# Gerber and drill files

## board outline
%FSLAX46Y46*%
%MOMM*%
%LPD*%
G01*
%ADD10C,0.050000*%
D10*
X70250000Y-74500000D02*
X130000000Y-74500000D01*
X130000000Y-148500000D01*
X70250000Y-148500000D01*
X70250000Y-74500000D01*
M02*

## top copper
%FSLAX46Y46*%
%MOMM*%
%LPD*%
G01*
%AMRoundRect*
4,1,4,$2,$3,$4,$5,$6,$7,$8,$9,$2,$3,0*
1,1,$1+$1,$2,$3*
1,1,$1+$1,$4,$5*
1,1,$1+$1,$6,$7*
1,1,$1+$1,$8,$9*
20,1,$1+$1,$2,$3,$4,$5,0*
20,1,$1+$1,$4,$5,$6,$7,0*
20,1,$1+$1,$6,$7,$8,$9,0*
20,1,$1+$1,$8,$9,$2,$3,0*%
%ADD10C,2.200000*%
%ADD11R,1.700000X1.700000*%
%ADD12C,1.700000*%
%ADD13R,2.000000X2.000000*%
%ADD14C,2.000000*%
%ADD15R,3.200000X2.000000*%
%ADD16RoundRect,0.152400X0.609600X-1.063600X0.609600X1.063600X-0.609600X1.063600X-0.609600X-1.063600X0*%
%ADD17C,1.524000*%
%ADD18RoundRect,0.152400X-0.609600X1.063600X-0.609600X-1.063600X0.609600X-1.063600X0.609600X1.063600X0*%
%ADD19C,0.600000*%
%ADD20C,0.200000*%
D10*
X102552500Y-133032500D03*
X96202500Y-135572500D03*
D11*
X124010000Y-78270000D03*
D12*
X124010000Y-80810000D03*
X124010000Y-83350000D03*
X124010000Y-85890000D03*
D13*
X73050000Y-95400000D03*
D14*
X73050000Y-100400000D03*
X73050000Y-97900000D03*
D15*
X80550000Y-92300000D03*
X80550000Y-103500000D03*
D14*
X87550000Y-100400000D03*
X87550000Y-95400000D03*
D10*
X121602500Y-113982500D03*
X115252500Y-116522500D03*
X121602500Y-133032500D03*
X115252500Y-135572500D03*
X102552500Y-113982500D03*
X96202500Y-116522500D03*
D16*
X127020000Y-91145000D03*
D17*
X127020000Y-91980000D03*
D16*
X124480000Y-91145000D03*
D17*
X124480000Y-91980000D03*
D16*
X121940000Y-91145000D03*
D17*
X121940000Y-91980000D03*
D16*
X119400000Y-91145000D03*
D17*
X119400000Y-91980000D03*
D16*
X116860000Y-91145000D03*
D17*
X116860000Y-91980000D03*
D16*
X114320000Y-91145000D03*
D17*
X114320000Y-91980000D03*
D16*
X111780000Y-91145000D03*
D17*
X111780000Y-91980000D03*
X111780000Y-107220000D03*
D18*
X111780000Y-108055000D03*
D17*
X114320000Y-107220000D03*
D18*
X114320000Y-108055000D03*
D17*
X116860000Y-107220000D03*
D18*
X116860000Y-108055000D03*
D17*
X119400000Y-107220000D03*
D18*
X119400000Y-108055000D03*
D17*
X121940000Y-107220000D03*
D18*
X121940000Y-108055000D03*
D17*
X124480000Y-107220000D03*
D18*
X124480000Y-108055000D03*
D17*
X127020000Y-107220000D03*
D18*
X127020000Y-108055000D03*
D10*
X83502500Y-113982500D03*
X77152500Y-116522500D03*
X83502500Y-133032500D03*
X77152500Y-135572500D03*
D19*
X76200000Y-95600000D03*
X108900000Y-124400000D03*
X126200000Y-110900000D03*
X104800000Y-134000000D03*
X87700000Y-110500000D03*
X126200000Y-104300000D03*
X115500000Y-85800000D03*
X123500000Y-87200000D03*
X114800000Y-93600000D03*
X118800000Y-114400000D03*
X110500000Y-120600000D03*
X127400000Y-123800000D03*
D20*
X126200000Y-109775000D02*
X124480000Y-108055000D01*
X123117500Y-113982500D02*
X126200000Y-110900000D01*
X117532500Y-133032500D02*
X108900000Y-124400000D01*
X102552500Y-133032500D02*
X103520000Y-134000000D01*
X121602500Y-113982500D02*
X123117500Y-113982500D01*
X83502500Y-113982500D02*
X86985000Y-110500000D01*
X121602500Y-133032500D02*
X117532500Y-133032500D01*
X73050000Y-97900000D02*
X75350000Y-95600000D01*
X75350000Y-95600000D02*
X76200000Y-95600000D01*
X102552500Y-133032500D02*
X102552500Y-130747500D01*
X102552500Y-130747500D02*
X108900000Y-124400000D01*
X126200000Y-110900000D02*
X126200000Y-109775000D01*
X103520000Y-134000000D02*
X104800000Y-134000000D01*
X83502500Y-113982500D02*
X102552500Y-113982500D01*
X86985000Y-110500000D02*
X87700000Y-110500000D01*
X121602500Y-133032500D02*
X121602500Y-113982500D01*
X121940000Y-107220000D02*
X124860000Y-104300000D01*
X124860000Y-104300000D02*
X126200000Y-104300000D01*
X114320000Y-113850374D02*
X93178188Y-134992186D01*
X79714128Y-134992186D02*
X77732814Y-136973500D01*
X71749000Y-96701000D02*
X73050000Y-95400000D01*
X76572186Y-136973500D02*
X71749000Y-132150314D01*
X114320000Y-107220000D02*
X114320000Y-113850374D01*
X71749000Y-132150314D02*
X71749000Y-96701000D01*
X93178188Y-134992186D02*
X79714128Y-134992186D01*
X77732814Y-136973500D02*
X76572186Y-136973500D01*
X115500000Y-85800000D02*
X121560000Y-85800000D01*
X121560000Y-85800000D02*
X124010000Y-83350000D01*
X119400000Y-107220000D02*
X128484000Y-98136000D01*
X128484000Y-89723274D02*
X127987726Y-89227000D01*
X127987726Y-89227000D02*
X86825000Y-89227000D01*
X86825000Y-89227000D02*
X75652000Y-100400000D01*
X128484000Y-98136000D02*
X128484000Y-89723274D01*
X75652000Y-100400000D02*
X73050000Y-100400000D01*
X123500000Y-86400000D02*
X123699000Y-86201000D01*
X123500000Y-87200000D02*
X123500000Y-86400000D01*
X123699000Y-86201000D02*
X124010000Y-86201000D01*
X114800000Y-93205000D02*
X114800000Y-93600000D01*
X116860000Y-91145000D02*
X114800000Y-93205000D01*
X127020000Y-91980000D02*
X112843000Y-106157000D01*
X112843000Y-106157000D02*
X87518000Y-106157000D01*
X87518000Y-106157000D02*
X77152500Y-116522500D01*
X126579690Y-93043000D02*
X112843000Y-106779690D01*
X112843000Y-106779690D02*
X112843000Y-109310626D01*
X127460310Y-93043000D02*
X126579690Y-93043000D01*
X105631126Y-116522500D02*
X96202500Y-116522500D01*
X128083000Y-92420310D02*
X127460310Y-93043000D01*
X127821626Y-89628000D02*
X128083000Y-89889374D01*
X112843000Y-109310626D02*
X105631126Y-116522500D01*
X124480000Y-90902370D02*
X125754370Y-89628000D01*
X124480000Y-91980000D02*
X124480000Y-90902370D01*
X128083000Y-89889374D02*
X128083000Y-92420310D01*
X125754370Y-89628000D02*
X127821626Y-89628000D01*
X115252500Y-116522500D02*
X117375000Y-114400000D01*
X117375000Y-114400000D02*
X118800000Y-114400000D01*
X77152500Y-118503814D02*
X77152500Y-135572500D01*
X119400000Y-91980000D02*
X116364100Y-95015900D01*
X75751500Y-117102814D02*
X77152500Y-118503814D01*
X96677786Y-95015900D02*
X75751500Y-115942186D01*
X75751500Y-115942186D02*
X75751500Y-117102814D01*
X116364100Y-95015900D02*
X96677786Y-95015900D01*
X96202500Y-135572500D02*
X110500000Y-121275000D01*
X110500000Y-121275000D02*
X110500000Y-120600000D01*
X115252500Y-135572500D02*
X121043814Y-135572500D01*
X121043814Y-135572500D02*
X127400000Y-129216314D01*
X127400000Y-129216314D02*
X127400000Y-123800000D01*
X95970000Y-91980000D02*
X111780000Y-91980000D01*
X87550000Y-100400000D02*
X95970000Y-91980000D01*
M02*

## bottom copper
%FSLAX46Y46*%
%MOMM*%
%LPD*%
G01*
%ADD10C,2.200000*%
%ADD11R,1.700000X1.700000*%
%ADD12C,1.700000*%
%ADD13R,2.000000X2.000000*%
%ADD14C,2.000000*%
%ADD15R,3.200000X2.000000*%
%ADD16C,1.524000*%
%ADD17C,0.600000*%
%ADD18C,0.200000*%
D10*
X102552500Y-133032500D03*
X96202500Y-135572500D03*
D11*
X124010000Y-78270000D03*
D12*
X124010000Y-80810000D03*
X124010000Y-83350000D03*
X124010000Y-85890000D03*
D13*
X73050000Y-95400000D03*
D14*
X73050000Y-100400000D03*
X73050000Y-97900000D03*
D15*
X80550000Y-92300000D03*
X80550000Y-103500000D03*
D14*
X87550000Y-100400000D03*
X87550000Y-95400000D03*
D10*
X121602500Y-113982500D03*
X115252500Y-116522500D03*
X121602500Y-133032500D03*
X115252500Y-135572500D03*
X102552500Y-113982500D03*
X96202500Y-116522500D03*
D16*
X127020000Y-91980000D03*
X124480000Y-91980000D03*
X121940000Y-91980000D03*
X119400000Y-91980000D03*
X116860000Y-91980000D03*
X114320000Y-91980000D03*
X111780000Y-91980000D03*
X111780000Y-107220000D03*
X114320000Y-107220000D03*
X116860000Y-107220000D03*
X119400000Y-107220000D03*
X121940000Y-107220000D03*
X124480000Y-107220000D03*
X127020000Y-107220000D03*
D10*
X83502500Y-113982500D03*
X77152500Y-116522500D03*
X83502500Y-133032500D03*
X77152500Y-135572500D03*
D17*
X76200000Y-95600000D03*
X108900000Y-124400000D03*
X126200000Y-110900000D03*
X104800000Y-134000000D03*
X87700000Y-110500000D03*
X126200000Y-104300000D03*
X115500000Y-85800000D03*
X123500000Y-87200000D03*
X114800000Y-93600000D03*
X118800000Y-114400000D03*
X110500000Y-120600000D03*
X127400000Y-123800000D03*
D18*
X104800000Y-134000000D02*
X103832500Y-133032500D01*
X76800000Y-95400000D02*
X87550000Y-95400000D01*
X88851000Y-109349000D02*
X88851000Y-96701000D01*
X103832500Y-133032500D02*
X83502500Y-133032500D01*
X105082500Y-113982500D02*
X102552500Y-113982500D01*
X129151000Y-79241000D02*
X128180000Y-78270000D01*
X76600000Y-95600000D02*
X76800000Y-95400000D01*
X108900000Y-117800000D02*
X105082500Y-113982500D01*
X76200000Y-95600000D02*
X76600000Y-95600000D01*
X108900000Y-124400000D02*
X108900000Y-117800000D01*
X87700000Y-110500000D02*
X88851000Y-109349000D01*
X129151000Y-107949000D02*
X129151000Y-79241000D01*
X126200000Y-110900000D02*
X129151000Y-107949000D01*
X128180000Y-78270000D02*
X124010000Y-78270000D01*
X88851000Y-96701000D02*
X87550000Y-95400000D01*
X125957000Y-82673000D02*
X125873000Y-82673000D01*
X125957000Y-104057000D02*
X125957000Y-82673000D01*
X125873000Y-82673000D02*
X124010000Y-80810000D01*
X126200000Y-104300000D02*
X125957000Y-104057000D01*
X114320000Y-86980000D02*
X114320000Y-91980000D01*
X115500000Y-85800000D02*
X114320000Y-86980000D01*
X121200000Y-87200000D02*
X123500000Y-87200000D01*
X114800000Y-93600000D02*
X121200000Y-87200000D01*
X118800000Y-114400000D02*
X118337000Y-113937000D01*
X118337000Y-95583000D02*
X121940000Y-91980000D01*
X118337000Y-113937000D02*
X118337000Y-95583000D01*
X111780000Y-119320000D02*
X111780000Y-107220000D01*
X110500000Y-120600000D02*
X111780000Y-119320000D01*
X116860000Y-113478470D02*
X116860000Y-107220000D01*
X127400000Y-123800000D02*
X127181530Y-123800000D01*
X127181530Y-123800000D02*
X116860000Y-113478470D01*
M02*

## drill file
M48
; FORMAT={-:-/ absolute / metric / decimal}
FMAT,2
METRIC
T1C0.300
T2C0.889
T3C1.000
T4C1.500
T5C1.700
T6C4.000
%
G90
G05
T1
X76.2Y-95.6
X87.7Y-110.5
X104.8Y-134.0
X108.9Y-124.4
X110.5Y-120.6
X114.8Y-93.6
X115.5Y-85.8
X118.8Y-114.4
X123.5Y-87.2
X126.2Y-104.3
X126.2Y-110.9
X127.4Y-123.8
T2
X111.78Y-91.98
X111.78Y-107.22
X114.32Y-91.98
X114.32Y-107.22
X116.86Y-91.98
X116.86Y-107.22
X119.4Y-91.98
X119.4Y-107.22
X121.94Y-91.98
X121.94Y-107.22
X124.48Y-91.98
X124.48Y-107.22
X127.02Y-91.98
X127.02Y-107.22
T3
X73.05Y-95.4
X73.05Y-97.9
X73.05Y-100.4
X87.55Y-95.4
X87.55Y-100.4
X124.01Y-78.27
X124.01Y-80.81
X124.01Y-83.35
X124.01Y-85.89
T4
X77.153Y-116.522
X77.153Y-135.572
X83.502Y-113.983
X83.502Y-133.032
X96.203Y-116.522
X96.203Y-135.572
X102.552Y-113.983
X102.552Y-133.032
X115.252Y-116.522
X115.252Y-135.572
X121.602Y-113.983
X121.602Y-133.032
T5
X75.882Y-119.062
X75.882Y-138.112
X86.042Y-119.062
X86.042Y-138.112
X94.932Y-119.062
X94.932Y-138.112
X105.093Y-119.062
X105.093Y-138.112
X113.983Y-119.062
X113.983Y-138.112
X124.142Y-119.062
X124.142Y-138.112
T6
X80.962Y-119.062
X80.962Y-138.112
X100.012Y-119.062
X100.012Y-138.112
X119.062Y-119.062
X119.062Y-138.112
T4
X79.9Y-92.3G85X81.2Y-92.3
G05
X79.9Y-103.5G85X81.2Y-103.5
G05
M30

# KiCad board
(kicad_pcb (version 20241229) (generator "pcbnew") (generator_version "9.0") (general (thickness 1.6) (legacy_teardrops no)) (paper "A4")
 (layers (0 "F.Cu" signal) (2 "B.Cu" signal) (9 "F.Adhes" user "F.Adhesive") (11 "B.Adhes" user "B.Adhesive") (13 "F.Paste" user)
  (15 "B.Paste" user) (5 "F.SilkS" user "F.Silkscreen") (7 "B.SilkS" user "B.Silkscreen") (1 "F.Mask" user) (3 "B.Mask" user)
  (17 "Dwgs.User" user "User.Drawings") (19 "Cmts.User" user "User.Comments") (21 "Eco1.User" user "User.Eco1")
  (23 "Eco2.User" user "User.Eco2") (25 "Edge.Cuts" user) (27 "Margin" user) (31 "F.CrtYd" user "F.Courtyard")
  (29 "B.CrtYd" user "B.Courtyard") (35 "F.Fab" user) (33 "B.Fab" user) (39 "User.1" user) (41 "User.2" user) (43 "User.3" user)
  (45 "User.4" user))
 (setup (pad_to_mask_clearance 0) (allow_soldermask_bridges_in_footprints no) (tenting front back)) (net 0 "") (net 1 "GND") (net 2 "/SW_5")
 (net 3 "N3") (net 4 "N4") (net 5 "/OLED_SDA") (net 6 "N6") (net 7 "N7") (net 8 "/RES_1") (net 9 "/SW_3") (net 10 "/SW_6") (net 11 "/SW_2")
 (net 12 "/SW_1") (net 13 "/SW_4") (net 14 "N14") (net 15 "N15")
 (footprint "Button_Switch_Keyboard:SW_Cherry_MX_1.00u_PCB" (layer "F.Cu") (at 102.5525 133.0325)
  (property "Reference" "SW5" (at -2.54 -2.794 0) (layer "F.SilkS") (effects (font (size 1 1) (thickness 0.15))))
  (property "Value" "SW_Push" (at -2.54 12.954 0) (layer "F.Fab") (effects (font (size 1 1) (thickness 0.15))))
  (pad "" np_thru_hole circle (at -7.62 5.08) (size 1.7 1.7) (drill 1.7) (layers "*.Cu" "*.Mask"))
  (pad "" np_thru_hole circle (at -2.54 5.08) (size 4 4) (drill 4) (layers "*.Cu" "*.Mask"))
  (pad "" np_thru_hole circle (at 2.54 5.08) (size 1.7 1.7) (drill 1.7) (layers "*.Cu" "*.Mask"))
  (pad "1" thru_hole circle (at 0 0) (size 2.2 2.2) (drill 1.5) (layers "*.Cu" "*.Mask") (remove_unused_layers no) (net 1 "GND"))
  (pad "2" thru_hole circle (at -6.35 2.54) (size 2.2 2.2) (drill 1.5) (layers "*.Cu" "*.Mask") (remove_unused_layers no) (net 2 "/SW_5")))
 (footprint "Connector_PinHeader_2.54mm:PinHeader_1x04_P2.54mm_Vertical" (layer "F.Cu") (at 124.01 78.27)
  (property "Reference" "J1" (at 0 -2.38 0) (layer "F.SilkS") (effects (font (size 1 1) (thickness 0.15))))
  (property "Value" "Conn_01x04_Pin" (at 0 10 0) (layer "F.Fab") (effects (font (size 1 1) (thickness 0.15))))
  (pad "1" thru_hole rect (at 0 0) (size 1.7 1.7) (drill 1) (layers "*.Cu" "*.Mask") (remove_unused_layers no) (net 1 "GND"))
  (pad "2" thru_hole circle (at 0 2.54) (size 1.7 1.7) (drill 1) (layers "*.Cu" "*.Mask") (remove_unused_layers no) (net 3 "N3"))
  (pad "3" thru_hole circle (at 0 5.08) (size 1.7 1.7) (drill 1) (layers "*.Cu" "*.Mask") (remove_unused_layers no) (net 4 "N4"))
  (pad "4" thru_hole circle (at 0 7.62) (size 1.7 1.7) (drill 1) (layers "*.Cu" "*.Mask") (remove_unused_layers no) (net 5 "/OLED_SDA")))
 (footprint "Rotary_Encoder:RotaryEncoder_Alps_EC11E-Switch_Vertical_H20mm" (layer "F.Cu") (at 73.05 95.4)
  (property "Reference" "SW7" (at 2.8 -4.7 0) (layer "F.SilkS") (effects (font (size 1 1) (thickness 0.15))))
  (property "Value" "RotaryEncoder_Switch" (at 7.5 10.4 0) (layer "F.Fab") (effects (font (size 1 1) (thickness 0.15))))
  (pad "A" thru_hole rect (at 0 0) (size 2 2) (drill 1) (layers "*.Cu" "*.Mask") (remove_unused_layers no) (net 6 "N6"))
  (pad "B" thru_hole circle (at 0 5) (size 2 2) (drill 1) (layers "*.Cu" "*.Mask") (remove_unused_layers no) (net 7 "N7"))
  (pad "C" thru_hole circle (at 0 2.5) (size 2 2) (drill 1) (layers "*.Cu" "*.Mask") (remove_unused_layers no) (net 1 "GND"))
  (pad "MP" thru_hole rect (at 7.5 -3.1) (size 3.2 2) (drill oval 2.8 1.5) (layers "*.Cu" "*.Mask") (remove_unused_layers no))
  (pad "MP" thru_hole rect (at 7.5 8.1) (size 3.2 2) (drill oval 2.8 1.5) (layers "*.Cu" "*.Mask") (remove_unused_layers no))
  (pad "S1" thru_hole circle (at 14.5 5) (size 2 2) (drill 1) (layers "*.Cu" "*.Mask") (remove_unused_layers no) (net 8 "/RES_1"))
  (pad "S2" thru_hole circle (at 14.5 0) (size 2 2) (drill 1) (layers "*.Cu" "*.Mask") (remove_unused_layers no) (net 1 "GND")))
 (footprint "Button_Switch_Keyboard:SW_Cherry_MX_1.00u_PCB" (layer "F.Cu") (at 121.6025 113.9825)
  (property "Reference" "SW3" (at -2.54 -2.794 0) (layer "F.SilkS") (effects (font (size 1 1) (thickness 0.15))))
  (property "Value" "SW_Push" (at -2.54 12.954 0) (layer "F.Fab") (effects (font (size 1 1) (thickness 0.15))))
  (pad "" np_thru_hole circle (at -7.62 5.08) (size 1.7 1.7) (drill 1.7) (layers "*.Cu" "*.Mask"))
  (pad "" np_thru_hole circle (at -2.54 5.08) (size 4 4) (drill 4) (layers "*.Cu" "*.Mask"))
  (pad "" np_thru_hole circle (at 2.54 5.08) (size 1.7 1.7) (drill 1.7) (layers "*.Cu" "*.Mask"))
  (pad "1" thru_hole circle (at 0 0) (size 2.2 2.2) (drill 1.5) (layers "*.Cu" "*.Mask") (remove_unused_layers no) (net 1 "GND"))
  (pad "2" thru_hole circle (at -6.35 2.54) (size 2.2 2.2) (drill 1.5) (layers "*.Cu" "*.Mask") (remove_unused_layers no) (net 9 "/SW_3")))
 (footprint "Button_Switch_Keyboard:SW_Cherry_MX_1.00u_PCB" (layer "F.Cu") (at 121.6025 133.0325)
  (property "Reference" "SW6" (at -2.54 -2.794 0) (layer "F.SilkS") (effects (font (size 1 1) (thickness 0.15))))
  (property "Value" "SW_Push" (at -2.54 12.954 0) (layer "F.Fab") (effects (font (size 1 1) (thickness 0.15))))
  (pad "" np_thru_hole circle (at -7.62 5.08) (size 1.7 1.7) (drill 1.7) (layers "*.Cu" "*.Mask"))
  (pad "" np_thru_hole circle (at -2.54 5.08) (size 4 4) (drill 4) (layers "*.Cu" "*.Mask"))
  (pad "" np_thru_hole circle (at 2.54 5.08) (size 1.7 1.7) (drill 1.7) (layers "*.Cu" "*.Mask"))
  (pad "1" thru_hole circle (at 0 0) (size 2.2 2.2) (drill 1.5) (layers "*.Cu" "*.Mask") (remove_unused_layers no) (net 1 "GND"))
  (pad "2" thru_hole circle (at -6.35 2.54) (size 2.2 2.2) (drill 1.5) (layers "*.Cu" "*.Mask") (remove_unused_layers no) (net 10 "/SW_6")))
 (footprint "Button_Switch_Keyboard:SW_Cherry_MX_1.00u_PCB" (layer "F.Cu") (at 102.5525 113.9825)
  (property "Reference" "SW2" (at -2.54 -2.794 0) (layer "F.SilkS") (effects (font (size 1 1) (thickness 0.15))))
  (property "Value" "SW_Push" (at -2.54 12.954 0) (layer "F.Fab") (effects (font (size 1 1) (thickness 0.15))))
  (pad "" np_thru_hole circle (at -7.62 5.08) (size 1.7 1.7) (drill 1.7) (layers "*.Cu" "*.Mask"))
  (pad "" np_thru_hole circle (at -2.54 5.08) (size 4 4) (drill 4) (layers "*.Cu" "*.Mask"))
  (pad "" np_thru_hole circle (at 2.54 5.08) (size 1.7 1.7) (drill 1.7) (layers "*.Cu" "*.Mask"))
  (pad "1" thru_hole circle (at 0 0) (size 2.2 2.2) (drill 1.5) (layers "*.Cu" "*.Mask") (remove_unused_layers no) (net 1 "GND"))
  (pad "2" thru_hole circle (at -6.35 2.54) (size 2.2 2.2) (drill 1.5) (layers "*.Cu" "*.Mask") (remove_unused_layers no) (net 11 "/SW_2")))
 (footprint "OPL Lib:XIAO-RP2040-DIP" (layer "F.Cu") (at 119.4 99.6 -90)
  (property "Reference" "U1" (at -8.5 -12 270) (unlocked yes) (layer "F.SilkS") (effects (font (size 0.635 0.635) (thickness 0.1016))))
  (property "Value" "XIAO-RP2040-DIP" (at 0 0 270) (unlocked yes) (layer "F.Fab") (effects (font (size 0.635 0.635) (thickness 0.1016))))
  (pad "1" smd roundrect (at -8.455 -7.62 90) (size 2.432 1.524) (layers "F.Cu" "F.Mask") (roundrect_rratio 0.1) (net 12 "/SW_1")
   (thermal_bridge_angle 45))
  (pad "1" thru_hole circle (at -7.62 -7.62 90) (size 1.524 1.524) (drill 0.889) (layers "*.Cu" "*.Mask") (remove_unused_layers no)
   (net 12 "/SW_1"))
  (pad "2" smd roundrect (at -8.455 -5.08 90) (size 2.432 1.524) (layers "F.Cu" "F.Mask") (roundrect_rratio 0.1) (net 11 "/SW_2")
   (thermal_bridge_angle 45))
  (pad "2" thru_hole circle (at -7.62 -5.08 90) (size 1.524 1.524) (drill 0.889) (layers "*.Cu" "*.Mask") (remove_unused_layers no)
   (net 11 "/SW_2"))
  (pad "3" smd roundrect (at -8.455 -2.54 90) (size 2.432 1.524) (layers "F.Cu" "F.Mask") (roundrect_rratio 0.1) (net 9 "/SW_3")
   (thermal_bridge_angle 45))
  (pad "3" thru_hole circle (at -7.62 -2.54 90) (size 1.524 1.524) (drill 0.889) (layers "*.Cu" "*.Mask") (remove_unused_layers no)
   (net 9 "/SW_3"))
  (pad "4" smd roundrect (at -8.455 0 90) (size 2.432 1.524) (layers "F.Cu" "F.Mask") (roundrect_rratio 0.1) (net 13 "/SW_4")
   (thermal_bridge_angle 45))
  (pad "4" thru_hole circle (at -7.62 0 90) (size 1.524 1.524) (drill 0.889) (layers "*.Cu" "*.Mask") (remove_unused_layers no)
   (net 13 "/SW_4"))
  (pad "5" smd roundrect (at -8.455 2.54 90) (size 2.432 1.524) (layers "F.Cu" "F.Mask") (roundrect_rratio 0.1) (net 5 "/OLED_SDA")
   (thermal_bridge_angle 45))
  (pad "5" thru_hole circle (at -7.62 2.54 90) (size 1.524 1.524) (drill 0.889) (layers "*.Cu" "*.Mask") (remove_unused_layers no)
   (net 5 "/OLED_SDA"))
  (pad "6" smd roundrect (at -8.455 5.08 90) (size 2.432 1.524) (layers "F.Cu" "F.Mask") (roundrect_rratio 0.1) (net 4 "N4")
   (thermal_bridge_angle 45))
  (pad "6" thru_hole circle (at -7.62 5.08 90) (size 1.524 1.524) (drill 0.889) (layers "*.Cu" "*.Mask") (remove_unused_layers no)
   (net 4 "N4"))
  (pad "7" smd roundrect (at -8.455 7.62 90) (size 2.432 1.524) (layers "F.Cu" "F.Mask") (roundrect_rratio 0.1) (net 8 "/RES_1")
   (thermal_bridge_angle 45))
  (pad "7" thru_hole circle (at -7.62 7.62 90) (size 1.524 1.524) (drill 0.889) (layers "*.Cu" "*.Mask") (remove_unused_layers no)
   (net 8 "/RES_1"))
  (pad "8" thru_hole circle (at 7.62 7.62 270) (size 1.524 1.524) (drill 0.889) (layers "*.Cu" "*.Mask") (remove_unused_layers no)
   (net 2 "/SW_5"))
  (pad "8" smd roundrect (at 8.455 7.62 270) (size 2.432 1.524) (layers "F.Cu" "F.Mask") (roundrect_rratio 0.1) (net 2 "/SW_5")
   (thermal_bridge_angle 45))
  (pad "9" thru_hole circle (at 7.62 5.08 270) (size 1.524 1.524) (drill 0.889) (layers "*.Cu" "*.Mask") (remove_unused_layers no)
   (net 6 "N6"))
  (pad "9" smd roundrect (at 8.455 5.08 270) (size 2.432 1.524) (layers "F.Cu" "F.Mask") (roundrect_rratio 0.1) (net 6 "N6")
   (thermal_bridge_angle 45))
  (pad "10" thru_hole circle (at 7.62 2.54 270) (size 1.524 1.524) (drill 0.889) (layers "*.Cu" "*.Mask") (remove_unused_layers no)
   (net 10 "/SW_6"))
  (pad "10" smd roundrect (at 8.455 2.54 270) (size 2.432 1.524) (layers "F.Cu" "F.Mask") (roundrect_rratio 0.1) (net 10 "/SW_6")
   (thermal_bridge_angle 45))
  (pad "11" thru_hole circle (at 7.62 0 270) (size 1.524 1.524) (drill 0.889) (layers "*.Cu" "*.Mask") (remove_unused_layers no)
   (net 7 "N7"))
  (pad "11" smd roundrect (at 8.455 0 270) (size 2.432 1.524) (layers "F.Cu" "F.Mask") (roundrect_rratio 0.1) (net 7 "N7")
   (thermal_bridge_angle 45))
  (pad "12" thru_hole circle (at 7.62 -2.54 270) (size 1.524 1.524) (drill 0.889) (layers "*.Cu" "*.Mask") (remove_unused_layers no)
   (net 3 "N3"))
  (pad "12" smd roundrect (at 8.455 -2.54 270) (size 2.432 1.524) (layers "F.Cu" "F.Mask") (roundrect_rratio 0.1) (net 3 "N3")
   (thermal_bridge_angle 45))
  (pad "13" thru_hole circle (at 7.62 -5.08 270) (size 1.524 1.524) (drill 0.889) (layers "*.Cu" "*.Mask") (remove_unused_layers no)
   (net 1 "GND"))
  (pad "13" smd roundrect (at 8.455 -5.08 270) (size 2.432 1.524) (layers "F.Cu" "F.Mask") (roundrect_rratio 0.1) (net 1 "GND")
   (thermal_bridge_angle 45))
  (pad "14" thru_hole circle (at 7.62 -7.62 270) (size 1.524 1.524) (drill 0.889) (layers "*.Cu" "*.Mask") (remove_unused_layers no)
   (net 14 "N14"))
  (pad "14" smd roundrect (at 8.455 -7.62 270) (size 2.432 1.524) (layers "F.Cu" "F.Mask") (roundrect_rratio 0.1) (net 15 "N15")
   (thermal_bridge_angle 45)))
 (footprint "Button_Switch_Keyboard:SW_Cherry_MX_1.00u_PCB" (layer "F.Cu") (at 83.5025 113.9825)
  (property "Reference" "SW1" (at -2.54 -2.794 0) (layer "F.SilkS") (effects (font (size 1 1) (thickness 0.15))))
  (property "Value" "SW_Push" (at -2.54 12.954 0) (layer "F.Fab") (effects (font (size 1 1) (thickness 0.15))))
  (pad "" np_thru_hole circle (at -7.62 5.08) (size 1.7 1.7) (drill 1.7) (layers "*.Cu" "*.Mask"))
  (pad "" np_thru_hole circle (at -2.54 5.08) (size 4 4) (drill 4) (layers "*.Cu" "*.Mask"))
  (pad "" np_thru_hole circle (at 2.54 5.08) (size 1.7 1.7) (drill 1.7) (layers "*.Cu" "*.Mask"))
  (pad "1" thru_hole circle (at 0 0) (size 2.2 2.2) (drill 1.5) (layers "*.Cu" "*.Mask") (remove_unused_layers no) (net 1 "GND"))
  (pad "2" thru_hole circle (at -6.35 2.54) (size 2.2 2.2) (drill 1.5) (layers "*.Cu" "*.Mask") (remove_unused_layers no) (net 12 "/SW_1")))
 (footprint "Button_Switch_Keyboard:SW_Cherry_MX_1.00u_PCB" (layer "F.Cu") (at 83.5025 133.0325)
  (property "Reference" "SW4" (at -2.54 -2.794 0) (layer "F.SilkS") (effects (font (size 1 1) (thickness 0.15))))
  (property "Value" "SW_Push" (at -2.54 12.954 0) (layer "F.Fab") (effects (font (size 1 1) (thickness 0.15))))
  (pad "" np_thru_hole circle (at -7.62 5.08) (size 1.7 1.7) (drill 1.7) (layers "*.Cu" "*.Mask"))
  (pad "" np_thru_hole circle (at -2.54 5.08) (size 4 4) (drill 4) (layers "*.Cu" "*.Mask"))
  (pad "" np_thru_hole circle (at 2.54 5.08) (size 1.7 1.7) (drill 1.7) (layers "*.Cu" "*.Mask"))
  (pad "1" thru_hole circle (at 0 0) (size 2.2 2.2) (drill 1.5) (layers "*.Cu" "*.Mask") (remove_unused_layers no) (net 1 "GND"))
  (pad "2" thru_hole circle (at -6.35 2.54) (size 2.2 2.2) (drill 1.5) (layers "*.Cu" "*.Mask") (remove_unused_layers no) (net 13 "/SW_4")))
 (gr_rect (start 70.25 74.5) (end 130 148.5) (stroke (width 0.05) (type default)) (fill no) (layer "Edge.Cuts"))
 (segment (start 126.2 109.775) (end 124.48 108.055) (width 0.2) (layer "F.Cu") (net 1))
 (segment (start 123.1175 113.9825) (end 126.2 110.9) (width 0.2) (layer "F.Cu") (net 1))
 (segment (start 117.5325 133.0325) (end 108.9 124.4) (width 0.2) (layer "F.Cu") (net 1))
 (segment (start 102.5525 133.0325) (end 103.52 134) (width 0.2) (layer "F.Cu") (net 1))
 (segment (start 121.6025 113.9825) (end 123.1175 113.9825) (width 0.2) (layer "F.Cu") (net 1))
 (segment (start 83.5025 113.9825) (end 86.985 110.5) (width 0.2) (layer "F.Cu") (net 1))
 (segment (start 121.6025 133.0325) (end 117.5325 133.0325) (width 0.2) (layer "F.Cu") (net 1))
 (segment (start 73.05 97.9) (end 75.35 95.6) (width 0.2) (layer "F.Cu") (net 1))
 (segment (start 75.35 95.6) (end 76.2 95.6) (width 0.2) (layer "F.Cu") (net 1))
 (segment (start 102.5525 133.0325) (end 102.5525 130.7475) (width 0.2) (layer "F.Cu") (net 1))
 (segment (start 102.5525 130.7475) (end 108.9 124.4) (width 0.2) (layer "F.Cu") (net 1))
 (segment (start 126.2 110.9) (end 126.2 109.775) (width 0.2) (layer "F.Cu") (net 1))
 (segment (start 103.52 134) (end 104.8 134) (width 0.2) (layer "F.Cu") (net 1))
 (segment (start 83.5025 113.9825) (end 102.5525 113.9825) (width 0.2) (layer "F.Cu") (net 1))
 (segment (start 86.985 110.5) (end 87.7 110.5) (width 0.2) (layer "F.Cu") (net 1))
 (segment (start 121.6025 133.0325) (end 121.6025 113.9825) (width 0.2) (layer "F.Cu") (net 1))
 (via (at 76.2 95.6) (size 0.6) (drill 0.3) (layers "F.Cu" "B.Cu") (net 1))
 (via (at 108.9 124.4) (size 0.6) (drill 0.3) (layers "F.Cu" "B.Cu") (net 1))
 (via (at 126.2 110.9) (size 0.6) (drill 0.3) (layers "F.Cu" "B.Cu") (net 1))
 (via (at 104.8 134) (size 0.6) (drill 0.3) (layers "F.Cu" "B.Cu") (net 1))
 (via (at 87.7 110.5) (size 0.6) (drill 0.3) (layers "F.Cu" "B.Cu") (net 1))
 (segment (start 104.8 134) (end 103.8325 133.0325) (width 0.2) (layer "B.Cu") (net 1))
 (segment (start 76.8 95.4) (end 87.55 95.4) (width 0.2) (layer "B.Cu") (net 1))
 (segment (start 88.851 109.349) (end 88.851 96.701) (width 0.2) (layer "B.Cu") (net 1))
 (segment (start 103.8325 133.0325) (end 83.5025 133.0325) (width 0.2) (layer "B.Cu") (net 1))
 (segment (start 105.0825 113.9825) (end 102.5525 113.9825) (width 0.2) (layer "B.Cu") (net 1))
 (segment (start 129.151 79.241) (end 128.18 78.27) (width 0.2) (layer "B.Cu") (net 1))
 (segment (start 76.6 95.6) (end 76.8 95.4) (width 0.2) (layer "B.Cu") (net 1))
 (segment (start 108.9 117.8) (end 105.0825 113.9825) (width 0.2) (layer "B.Cu") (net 1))
 (segment (start 76.2 95.6) (end 76.6 95.6) (width 0.2) (layer "B.Cu") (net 1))
 (segment (start 108.9 124.4) (end 108.9 117.8) (width 0.2) (layer "B.Cu") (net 1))
 (segment (start 87.7 110.5) (end 88.851 109.349) (width 0.2) (layer "B.Cu") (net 1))
 (segment (start 129.151 107.949) (end 129.151 79.241) (width 0.2) (layer "B.Cu") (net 1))
 (segment (start 126.2 110.9) (end 129.151 107.949) (width 0.2) (layer "B.Cu") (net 1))
 (segment (start 128.18 78.27) (end 124.01 78.27) (width 0.2) (layer "B.Cu") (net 1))
 (segment (start 88.851 96.701) (end 87.55 95.4) (width 0.2) (layer "B.Cu") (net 1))
 (segment (start 121.94 107.22) (end 124.86 104.3) (width 0.2) (layer "F.Cu") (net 3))
 (segment (start 124.86 104.3) (end 126.2 104.3) (width 0.2) (layer "F.Cu") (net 3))
 (via (at 126.2 104.3) (size 0.6) (drill 0.3) (layers "F.Cu" "B.Cu") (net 3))
 (segment (start 125.957 82.673) (end 125.873 82.673) (width 0.2) (layer "B.Cu") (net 3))
 (segment (start 125.957 104.057) (end 125.957 82.673) (width 0.2) (layer "B.Cu") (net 3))
 (segment (start 125.873 82.673) (end 124.01 80.81) (width 0.2) (layer "B.Cu") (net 3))
 (segment (start 126.2 104.3) (end 125.957 104.057) (width 0.2) (layer "B.Cu") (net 3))
 (segment (start 114.32 113.850374) (end 93.178188 134.992186) (width 0.2) (layer "F.Cu") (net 6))
 (segment (start 79.714128 134.992186) (end 77.732814 136.9735) (width 0.2) (layer "F.Cu") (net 6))
 (segment (start 71.749 96.701) (end 73.05 95.4) (width 0.2) (layer "F.Cu") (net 6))
 (segment (start 76.572186 136.9735) (end 71.749 132.150314) (width 0.2) (layer "F.Cu") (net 6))
 (segment (start 114.32 107.22) (end 114.32 113.850374) (width 0.2) (layer "F.Cu") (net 6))
 (segment (start 71.749 132.150314) (end 71.749 96.701) (width 0.2) (layer "F.Cu") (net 6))
 (segment (start 93.178188 134.992186) (end 79.714128 134.992186) (width 0.2) (layer "F.Cu") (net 6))
 (segment (start 77.732814 136.9735) (end 76.572186 136.9735) (width 0.2) (layer "F.Cu") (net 6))
 (segment (start 115.5 85.8) (end 121.56 85.8) (width 0.2) (layer "F.Cu") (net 4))
 (segment (start 121.56 85.8) (end 124.01 83.35) (width 0.2) (layer "F.Cu") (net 4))
 (via (at 115.5 85.8) (size 0.6) (drill 0.3) (layers "F.Cu" "B.Cu") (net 4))
 (segment (start 114.32 86.98) (end 114.32 91.98) (width 0.2) (layer "B.Cu") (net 4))
 (segment (start 115.5 85.8) (end 114.32 86.98) (width 0.2) (layer "B.Cu") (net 4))
 (segment (start 119.4 107.22) (end 128.484 98.136) (width 0.2) (layer "F.Cu") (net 7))
 (segment (start 128.484 89.723274) (end 127.987726 89.227) (width 0.2) (layer "F.Cu") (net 7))
 (segment (start 127.987726 89.227) (end 86.825 89.227) (width 0.2) (layer "F.Cu") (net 7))
 (segment (start 86.825 89.227) (end 75.652 100.4) (width 0.2) (layer "F.Cu") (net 7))
 (segment (start 128.484 98.136) (end 128.484 89.723274) (width 0.2) (layer "F.Cu") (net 7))
 (segment (start 75.652 100.4) (end 73.05 100.4) (width 0.2) (layer "F.Cu") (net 7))
 (segment (start 123.5 86.4) (end 123.699 86.201) (width 0.2) (layer "F.Cu") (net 5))
 (segment (start 123.5 87.2) (end 123.5 86.4) (width 0.2) (layer "F.Cu") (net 5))
 (segment (start 123.699 86.201) (end 124.01 86.201) (width 0.2) (layer "F.Cu") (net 5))
 (segment (start 114.8 93.205) (end 114.8 93.6) (width 0.2) (layer "F.Cu") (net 5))
 (segment (start 116.86 91.145) (end 114.8 93.205) (width 0.2) (layer "F.Cu") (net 5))
 (via (at 123.5 87.2) (size 0.6) (drill 0.3) (layers "F.Cu" "B.Cu") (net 5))
 (via (at 114.8 93.6) (size 0.6) (drill 0.3) (layers "F.Cu" "B.Cu") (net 5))
 (segment (start 121.2 87.2) (end 123.5 87.2) (width 0.2) (layer "B.Cu") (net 5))
 (segment (start 114.8 93.6) (end 121.2 87.2) (width 0.2) (layer "B.Cu") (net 5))
 (segment (start 127.02 91.98) (end 112.843 106.157) (width 0.2) (layer "F.Cu") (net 12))
 (segment (start 112.843 106.157) (end 87.518 106.157) (width 0.2) (layer "F.Cu") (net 12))
 (segment (start 87.518 106.157) (end 77.1525 116.5225) (width 0.2) (layer "F.Cu") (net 12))
 (segment (start 126.57969 93.043) (end 112.843 106.77969) (width 0.2) (layer "F.Cu") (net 11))
 (segment (start 112.843 106.77969) (end 112.843 109.310626) (width 0.2) (layer "F.Cu") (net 11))
 (segment (start 127.46031 93.043) (end 126.57969 93.043) (width 0.2) (layer "F.Cu") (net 11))
 (segment (start 105.631126 116.5225) (end 96.2025 116.5225) (width 0.2) (layer "F.Cu") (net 11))
 (segment (start 128.083 92.42031) (end 127.46031 93.043) (width 0.2) (layer "F.Cu") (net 11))
 (segment (start 127.821626 89.628) (end 128.083 89.889374) (width 0.2) (layer "F.Cu") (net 11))
 (segment (start 112.843 109.310626) (end 105.631126 116.5225) (width 0.2) (layer "F.Cu") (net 11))
 (segment (start 124.48 90.90237) (end 125.75437 89.628) (width 0.2) (layer "F.Cu") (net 11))
 (segment (start 124.48 91.98) (end 124.48 90.90237) (width 0.2) (layer "F.Cu") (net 11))
 (segment (start 128.083 89.889374) (end 128.083 92.42031) (width 0.2) (layer "F.Cu") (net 11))
 (segment (start 125.75437 89.628) (end 127.821626 89.628) (width 0.2) (layer "F.Cu") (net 11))
 (segment (start 115.2525 116.5225) (end 117.375 114.4) (width 0.2) (layer "F.Cu") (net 9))
 (segment (start 117.375 114.4) (end 118.8 114.4) (width 0.2) (layer "F.Cu") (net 9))
 (via (at 118.8 114.4) (size 0.6) (drill 0.3) (layers "F.Cu" "B.Cu") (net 9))
 (segment (start 118.8 114.4) (end 118.337 113.937) (width 0.2) (layer "B.Cu") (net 9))
 (segment (start 118.337 95.583) (end 121.94 91.98) (width 0.2) (layer "B.Cu") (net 9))
 (segment (start 118.337 113.937) (end 118.337 95.583) (width 0.2) (layer "B.Cu") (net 9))
 (segment (start 77.1525 118.503814) (end 77.1525 135.5725) (width 0.2) (layer "F.Cu") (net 13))
 (segment (start 119.4 91.98) (end 116.3641 95.0159) (width 0.2) (layer "F.Cu") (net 13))
 (segment (start 75.7515 117.102814) (end 77.1525 118.503814) (width 0.2) (layer "F.Cu") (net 13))
 (segment (start 96.677786 95.0159) (end 75.7515 115.942186) (width 0.2) (layer "F.Cu") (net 13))
 (segment (start 75.7515 115.942186) (end 75.7515 117.102814) (width 0.2) (layer "F.Cu") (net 13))
 (segment (start 116.3641 95.0159) (end 96.677786 95.0159) (width 0.2) (layer "F.Cu") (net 13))
 (segment (start 96.2025 135.5725) (end 110.5 121.275) (width 0.2) (layer "F.Cu") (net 2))
 (segment (start 110.5 121.275) (end 110.5 120.6) (width 0.2) (layer "F.Cu") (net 2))
 (via (at 110.5 120.6) (size 0.6) (drill 0.3) (layers "F.Cu" "B.Cu") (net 2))
 (segment (start 111.78 119.32) (end 111.78 107.22) (width 0.2) (layer "B.Cu") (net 2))
 (segment (start 110.5 120.6) (end 111.78 119.32) (width 0.2) (layer "B.Cu") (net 2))
 (segment (start 115.2525 135.5725) (end 121.043814 135.5725) (width 0.2) (layer "F.Cu") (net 10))
 (segment (start 121.043814 135.5725) (end 127.4 129.216314) (width 0.2) (layer "F.Cu") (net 10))
 (segment (start 127.4 129.216314) (end 127.4 123.8) (width 0.2) (layer "F.Cu") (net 10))
 (via (at 127.4 123.8) (size 0.6) (drill 0.3) (layers "F.Cu" "B.Cu") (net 10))
 (segment (start 116.86 113.47847) (end 116.86 107.22) (width 0.2) (layer "B.Cu") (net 10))
 (segment (start 127.4 123.8) (end 127.18153 123.8) (width 0.2) (layer "B.Cu") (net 10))
 (segment (start 127.18153 123.8) (end 116.86 113.47847) (width 0.2) (layer "B.Cu") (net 10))
 (segment (start 95.97 91.98) (end 111.78 91.98) (width 0.2) (layer "F.Cu") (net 8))
 (segment (start 87.55 100.4) (end 95.97 91.98) (width 0.2) (layer "F.Cu") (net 8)))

